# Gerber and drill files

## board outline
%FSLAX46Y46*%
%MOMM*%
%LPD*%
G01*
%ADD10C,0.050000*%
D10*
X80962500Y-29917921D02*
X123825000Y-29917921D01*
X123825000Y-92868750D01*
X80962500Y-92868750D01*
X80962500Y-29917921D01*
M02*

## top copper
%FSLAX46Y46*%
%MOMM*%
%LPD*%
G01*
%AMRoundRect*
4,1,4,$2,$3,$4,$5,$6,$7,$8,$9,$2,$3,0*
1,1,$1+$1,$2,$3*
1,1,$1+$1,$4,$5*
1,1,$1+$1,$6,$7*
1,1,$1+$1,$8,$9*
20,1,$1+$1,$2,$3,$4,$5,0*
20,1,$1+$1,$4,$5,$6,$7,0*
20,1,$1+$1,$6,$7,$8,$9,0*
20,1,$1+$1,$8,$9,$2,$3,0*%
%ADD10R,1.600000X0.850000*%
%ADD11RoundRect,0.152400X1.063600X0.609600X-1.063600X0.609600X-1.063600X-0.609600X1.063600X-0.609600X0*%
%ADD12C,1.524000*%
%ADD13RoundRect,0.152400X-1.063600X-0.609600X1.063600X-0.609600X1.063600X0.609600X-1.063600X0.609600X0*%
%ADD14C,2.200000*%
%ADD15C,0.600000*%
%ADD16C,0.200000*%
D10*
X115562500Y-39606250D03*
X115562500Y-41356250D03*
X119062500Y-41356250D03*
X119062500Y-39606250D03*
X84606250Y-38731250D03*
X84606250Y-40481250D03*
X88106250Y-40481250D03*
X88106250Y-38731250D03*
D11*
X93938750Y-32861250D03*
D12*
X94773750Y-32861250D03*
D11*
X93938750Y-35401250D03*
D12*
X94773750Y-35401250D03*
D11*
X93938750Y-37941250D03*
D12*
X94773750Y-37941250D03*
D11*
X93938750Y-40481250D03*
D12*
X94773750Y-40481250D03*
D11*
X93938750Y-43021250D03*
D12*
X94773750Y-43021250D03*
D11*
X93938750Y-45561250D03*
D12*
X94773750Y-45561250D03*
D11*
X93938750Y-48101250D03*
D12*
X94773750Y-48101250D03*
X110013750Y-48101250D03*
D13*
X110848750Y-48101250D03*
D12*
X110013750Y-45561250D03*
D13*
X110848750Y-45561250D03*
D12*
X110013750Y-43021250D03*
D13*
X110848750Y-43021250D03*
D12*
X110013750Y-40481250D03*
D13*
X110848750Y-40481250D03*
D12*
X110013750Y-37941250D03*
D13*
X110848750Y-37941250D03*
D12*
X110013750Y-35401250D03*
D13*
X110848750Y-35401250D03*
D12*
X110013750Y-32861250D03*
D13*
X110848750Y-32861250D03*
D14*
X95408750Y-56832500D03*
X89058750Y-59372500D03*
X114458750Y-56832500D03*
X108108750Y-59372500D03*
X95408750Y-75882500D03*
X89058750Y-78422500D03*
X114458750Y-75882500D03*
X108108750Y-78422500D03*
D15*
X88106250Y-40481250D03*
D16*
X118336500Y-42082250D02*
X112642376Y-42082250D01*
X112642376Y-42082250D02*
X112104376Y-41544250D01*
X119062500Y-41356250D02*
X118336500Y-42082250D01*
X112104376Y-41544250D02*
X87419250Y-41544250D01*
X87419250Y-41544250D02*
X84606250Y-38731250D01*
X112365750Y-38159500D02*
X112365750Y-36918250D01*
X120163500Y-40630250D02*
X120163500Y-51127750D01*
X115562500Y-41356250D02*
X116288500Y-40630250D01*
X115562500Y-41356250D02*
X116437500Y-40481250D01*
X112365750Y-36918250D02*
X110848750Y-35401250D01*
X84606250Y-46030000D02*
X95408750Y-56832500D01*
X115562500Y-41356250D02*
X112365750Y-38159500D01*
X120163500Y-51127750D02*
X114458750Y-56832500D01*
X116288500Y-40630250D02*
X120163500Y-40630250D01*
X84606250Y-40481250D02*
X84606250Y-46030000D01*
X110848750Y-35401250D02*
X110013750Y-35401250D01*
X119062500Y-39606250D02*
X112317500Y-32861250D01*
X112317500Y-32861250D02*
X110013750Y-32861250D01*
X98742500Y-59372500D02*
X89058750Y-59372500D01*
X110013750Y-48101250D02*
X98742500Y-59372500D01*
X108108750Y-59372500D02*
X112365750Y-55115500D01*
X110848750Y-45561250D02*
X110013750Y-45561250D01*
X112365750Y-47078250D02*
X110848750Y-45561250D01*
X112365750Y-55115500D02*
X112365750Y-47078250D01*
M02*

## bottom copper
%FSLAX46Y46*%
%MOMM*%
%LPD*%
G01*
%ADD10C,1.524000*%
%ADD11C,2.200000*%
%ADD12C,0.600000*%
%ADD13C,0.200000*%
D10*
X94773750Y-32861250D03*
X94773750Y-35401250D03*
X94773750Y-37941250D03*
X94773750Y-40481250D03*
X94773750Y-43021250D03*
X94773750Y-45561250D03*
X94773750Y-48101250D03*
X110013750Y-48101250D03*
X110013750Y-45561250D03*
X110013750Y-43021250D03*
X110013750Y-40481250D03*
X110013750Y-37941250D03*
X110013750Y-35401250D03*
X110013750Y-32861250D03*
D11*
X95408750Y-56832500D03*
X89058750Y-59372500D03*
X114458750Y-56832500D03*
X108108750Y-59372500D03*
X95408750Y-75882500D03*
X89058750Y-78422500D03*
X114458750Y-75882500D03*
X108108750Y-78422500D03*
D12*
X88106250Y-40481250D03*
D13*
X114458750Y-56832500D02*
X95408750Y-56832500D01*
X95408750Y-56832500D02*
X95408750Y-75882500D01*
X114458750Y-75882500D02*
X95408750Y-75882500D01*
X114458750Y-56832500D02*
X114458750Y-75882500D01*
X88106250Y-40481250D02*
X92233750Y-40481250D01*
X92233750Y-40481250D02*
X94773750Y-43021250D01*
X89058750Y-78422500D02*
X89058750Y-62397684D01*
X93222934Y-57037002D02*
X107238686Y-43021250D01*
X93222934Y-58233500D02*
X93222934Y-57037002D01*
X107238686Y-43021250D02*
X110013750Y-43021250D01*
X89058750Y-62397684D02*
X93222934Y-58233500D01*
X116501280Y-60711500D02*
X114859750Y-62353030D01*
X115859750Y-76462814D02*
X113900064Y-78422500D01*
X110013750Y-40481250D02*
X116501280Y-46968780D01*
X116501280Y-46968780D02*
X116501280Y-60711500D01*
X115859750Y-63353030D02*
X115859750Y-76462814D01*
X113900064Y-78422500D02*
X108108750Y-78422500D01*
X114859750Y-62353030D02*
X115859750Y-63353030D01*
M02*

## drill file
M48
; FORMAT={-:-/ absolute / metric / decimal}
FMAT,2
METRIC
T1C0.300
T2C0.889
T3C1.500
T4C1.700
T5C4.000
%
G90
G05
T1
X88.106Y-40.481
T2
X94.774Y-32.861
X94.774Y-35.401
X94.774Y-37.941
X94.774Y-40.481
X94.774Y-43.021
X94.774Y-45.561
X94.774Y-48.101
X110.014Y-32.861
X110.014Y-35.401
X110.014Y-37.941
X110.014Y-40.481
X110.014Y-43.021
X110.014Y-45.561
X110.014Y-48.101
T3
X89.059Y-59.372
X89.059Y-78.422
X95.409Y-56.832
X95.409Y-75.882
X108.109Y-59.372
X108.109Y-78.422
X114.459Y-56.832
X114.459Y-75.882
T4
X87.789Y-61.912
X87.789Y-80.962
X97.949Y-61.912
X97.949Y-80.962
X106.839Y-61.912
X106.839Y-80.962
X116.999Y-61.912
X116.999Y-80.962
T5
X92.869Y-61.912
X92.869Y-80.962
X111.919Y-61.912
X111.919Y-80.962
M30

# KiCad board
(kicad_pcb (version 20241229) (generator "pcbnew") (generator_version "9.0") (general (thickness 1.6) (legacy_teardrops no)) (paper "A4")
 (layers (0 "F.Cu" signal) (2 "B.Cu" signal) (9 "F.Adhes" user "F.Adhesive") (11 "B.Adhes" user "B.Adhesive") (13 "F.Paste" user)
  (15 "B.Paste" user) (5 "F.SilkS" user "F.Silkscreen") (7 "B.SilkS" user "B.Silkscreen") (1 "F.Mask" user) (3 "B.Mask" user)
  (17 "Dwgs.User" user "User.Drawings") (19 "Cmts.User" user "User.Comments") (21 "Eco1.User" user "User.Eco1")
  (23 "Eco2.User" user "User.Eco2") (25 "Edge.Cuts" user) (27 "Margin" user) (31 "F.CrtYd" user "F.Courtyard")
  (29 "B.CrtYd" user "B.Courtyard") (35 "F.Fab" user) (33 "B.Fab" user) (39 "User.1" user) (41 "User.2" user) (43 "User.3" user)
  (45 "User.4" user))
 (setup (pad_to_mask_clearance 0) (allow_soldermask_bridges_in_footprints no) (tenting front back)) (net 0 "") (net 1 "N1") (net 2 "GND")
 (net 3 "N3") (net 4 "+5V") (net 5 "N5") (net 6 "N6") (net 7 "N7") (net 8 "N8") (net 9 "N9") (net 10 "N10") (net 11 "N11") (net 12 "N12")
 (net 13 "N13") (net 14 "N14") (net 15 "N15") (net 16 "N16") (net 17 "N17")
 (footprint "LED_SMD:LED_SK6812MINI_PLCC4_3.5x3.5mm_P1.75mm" (layer "F.Cu") (at 117.3125 40.48125)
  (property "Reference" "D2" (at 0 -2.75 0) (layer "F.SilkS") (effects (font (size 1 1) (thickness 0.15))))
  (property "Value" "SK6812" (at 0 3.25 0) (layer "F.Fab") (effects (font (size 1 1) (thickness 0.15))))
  (pad "1" smd rect (at -1.75 -0.875) (size 1.6 0.85) (layers "F.Cu" "F.Mask" "F.Paste") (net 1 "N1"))
  (pad "2" smd rect (at -1.75 0.875) (size 1.6 0.85) (layers "F.Cu" "F.Mask" "F.Paste") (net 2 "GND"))
  (pad "3" smd rect (at 1.75 0.875) (size 1.6 0.85) (layers "F.Cu" "F.Mask" "F.Paste") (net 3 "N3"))
  (pad "4" smd rect (at 1.75 -0.875) (size 1.6 0.85) (layers "F.Cu" "F.Mask" "F.Paste") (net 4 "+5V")))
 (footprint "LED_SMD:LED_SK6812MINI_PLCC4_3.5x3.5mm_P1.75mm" (layer "F.Cu") (at 86.35625 39.60625)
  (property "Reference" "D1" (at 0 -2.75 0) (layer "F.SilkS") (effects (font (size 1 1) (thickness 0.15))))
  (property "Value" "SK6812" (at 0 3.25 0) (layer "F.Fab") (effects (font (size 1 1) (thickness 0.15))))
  (pad "1" smd rect (at -1.75 -0.875) (size 1.6 0.85) (layers "F.Cu" "F.Mask" "F.Paste") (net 3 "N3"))
  (pad "2" smd rect (at -1.75 0.875) (size 1.6 0.85) (layers "F.Cu" "F.Mask" "F.Paste") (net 2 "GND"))
  (pad "3" smd rect (at 1.75 0.875) (size 1.6 0.85) (layers "F.Cu" "F.Mask" "F.Paste") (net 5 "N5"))
  (pad "4" smd rect (at 1.75 -0.875) (size 1.6 0.85) (layers "F.Cu" "F.Mask" "F.Paste") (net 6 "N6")))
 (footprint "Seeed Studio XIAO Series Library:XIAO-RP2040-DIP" (layer "F.Cu") (at 102.39375 40.48125)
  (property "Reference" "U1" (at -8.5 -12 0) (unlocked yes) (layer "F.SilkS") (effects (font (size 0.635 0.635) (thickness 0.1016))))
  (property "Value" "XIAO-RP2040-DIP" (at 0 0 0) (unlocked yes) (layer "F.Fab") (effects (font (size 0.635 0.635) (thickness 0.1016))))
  (pad "1" smd roundrect (at -8.455 -7.62 180) (size 2.432 1.524) (layers "F.Cu" "F.Mask") (roundrect_rratio 0.1) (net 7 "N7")
   (thermal_bridge_angle 45))
  (pad "1" thru_hole circle (at -7.62 -7.62 180) (size 1.524 1.524) (drill 0.889) (layers "*.Cu" "*.Mask") (remove_unused_layers no)
   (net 7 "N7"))
  (pad "2" smd roundrect (at -8.455 -5.08 180) (size 2.432 1.524) (layers "F.Cu" "F.Mask") (roundrect_rratio 0.1) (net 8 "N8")
   (thermal_bridge_angle 45))
  (pad "2" thru_hole circle (at -7.62 -5.08 180) (size 1.524 1.524) (drill 0.889) (layers "*.Cu" "*.Mask") (remove_unused_layers no)
   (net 8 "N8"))
  (pad "3" smd roundrect (at -8.455 -2.54 180) (size 2.432 1.524) (layers "F.Cu" "F.Mask") (roundrect_rratio 0.1) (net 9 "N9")
   (thermal_bridge_angle 45))
  (pad "3" thru_hole circle (at -7.62 -2.54 180) (size 1.524 1.524) (drill 0.889) (layers "*.Cu" "*.Mask") (remove_unused_layers no)
   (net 9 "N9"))
  (pad "4" smd roundrect (at -8.455 0 180) (size 2.432 1.524) (layers "F.Cu" "F.Mask") (roundrect_rratio 0.1) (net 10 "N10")
   (thermal_bridge_angle 45))
  (pad "4" thru_hole circle (at -7.62 0 180) (size 1.524 1.524) (drill 0.889) (layers "*.Cu" "*.Mask") (remove_unused_layers no)
   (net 10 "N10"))
  (pad "5" smd roundrect (at -8.455 2.54 180) (size 2.432 1.524) (layers "F.Cu" "F.Mask") (roundrect_rratio 0.1) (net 5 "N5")
   (thermal_bridge_angle 45))
  (pad "5" thru_hole circle (at -7.62 2.54 180) (size 1.524 1.524) (drill 0.889) (layers "*.Cu" "*.Mask") (remove_unused_layers no)
   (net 5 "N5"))
  (pad "6" smd roundrect (at -8.455 5.08 180) (size 2.432 1.524) (layers "F.Cu" "F.Mask") (roundrect_rratio 0.1) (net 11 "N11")
   (thermal_bridge_angle 45))
  (pad "6" thru_hole circle (at -7.62 5.08 180) (size 1.524 1.524) (drill 0.889) (layers "*.Cu" "*.Mask") (remove_unused_layers no)
   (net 11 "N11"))
  (pad "7" smd roundrect (at -8.455 7.62 180) (size 2.432 1.524) (layers "F.Cu" "F.Mask") (roundrect_rratio 0.1) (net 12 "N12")
   (thermal_bridge_angle 45))
  (pad "7" thru_hole circle (at -7.62 7.62 180) (size 1.524 1.524) (drill 0.889) (layers "*.Cu" "*.Mask") (remove_unused_layers no)
   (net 12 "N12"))
  (pad "8" thru_hole circle (at 7.62 7.62) (size 1.524 1.524) (drill 0.889) (layers "*.Cu" "*.Mask") (remove_unused_layers no)
   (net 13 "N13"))
  (pad "8" smd roundrect (at 8.455 7.62) (size 2.432 1.524) (layers "F.Cu" "F.Mask") (roundrect_rratio 0.1) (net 13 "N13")
   (thermal_bridge_angle 45))
  (pad "9" thru_hole circle (at 7.62 5.08) (size 1.524 1.524) (drill 0.889) (layers "*.Cu" "*.Mask") (remove_unused_layers no)
   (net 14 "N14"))
  (pad "9" smd roundrect (at 8.455 5.08) (size 2.432 1.524) (layers "F.Cu" "F.Mask") (roundrect_rratio 0.1) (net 14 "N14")
   (thermal_bridge_angle 45))
  (pad "10" thru_hole circle (at 7.62 2.54) (size 1.524 1.524) (drill 0.889) (layers "*.Cu" "*.Mask") (remove_unused_layers no)
   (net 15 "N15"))
  (pad "10" smd roundrect (at 8.455 2.54) (size 2.432 1.524) (layers "F.Cu" "F.Mask") (roundrect_rratio 0.1) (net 15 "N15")
   (thermal_bridge_angle 45))
  (pad "11" thru_hole circle (at 7.62 0) (size 1.524 1.524) (drill 0.889) (layers "*.Cu" "*.Mask") (remove_unused_layers no) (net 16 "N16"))
  (pad "11" smd roundrect (at 8.455 0) (size 2.432 1.524) (layers "F.Cu" "F.Mask") (roundrect_rratio 0.1) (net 16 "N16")
   (thermal_bridge_angle 45))
  (pad "12" thru_hole circle (at 7.62 -2.54) (size 1.524 1.524) (drill 0.889) (layers "*.Cu" "*.Mask") (remove_unused_layers no)
   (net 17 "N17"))
  (pad "12" smd roundrect (at 8.455 -2.54) (size 2.432 1.524) (layers "F.Cu" "F.Mask") (roundrect_rratio 0.1) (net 17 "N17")
   (thermal_bridge_angle 45))
  (pad "13" thru_hole circle (at 7.62 -5.08) (size 1.524 1.524) (drill 0.889) (layers "*.Cu" "*.Mask") (remove_unused_layers no)
   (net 2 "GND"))
  (pad "13" smd roundrect (at 8.455 -5.08) (size 2.432 1.524) (layers "F.Cu" "F.Mask") (roundrect_rratio 0.1) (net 2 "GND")
   (thermal_bridge_angle 45))
  (pad "14" thru_hole circle (at 7.62 -7.62) (size 1.524 1.524) (drill 0.889) (layers "*.Cu" "*.Mask") (remove_unused_layers no)
   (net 4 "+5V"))
  (pad "14" smd roundrect (at 8.455 -7.62) (size 2.432 1.524) (layers "F.Cu" "F.Mask") (roundrect_rratio 0.1) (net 4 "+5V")
   (thermal_bridge_angle 45)))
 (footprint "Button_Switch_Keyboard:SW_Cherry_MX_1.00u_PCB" (layer "F.Cu") (at 95.40875 56.8325)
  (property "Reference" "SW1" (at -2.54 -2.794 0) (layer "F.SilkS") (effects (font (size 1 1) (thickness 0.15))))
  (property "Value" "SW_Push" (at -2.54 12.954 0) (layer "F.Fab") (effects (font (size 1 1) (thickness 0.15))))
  (pad "" np_thru_hole circle (at -7.62 5.08) (size 1.7 1.7) (drill 1.7) (layers "*.Cu" "*.Mask"))
  (pad "" np_thru_hole circle (at -2.54 5.08) (size 4 4) (drill 4) (layers "*.Cu" "*.Mask"))
  (pad "" np_thru_hole circle (at 2.54 5.08) (size 1.7 1.7) (drill 1.7) (layers "*.Cu" "*.Mask"))
  (pad "1" thru_hole circle (at 0 0) (size 2.2 2.2) (drill 1.5) (layers "*.Cu" "*.Mask") (remove_unused_layers no) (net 2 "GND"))
  (pad "2" thru_hole circle (at -6.35 2.54) (size 2.2 2.2) (drill 1.5) (layers "*.Cu" "*.Mask") (remove_unused_layers no) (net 13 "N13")))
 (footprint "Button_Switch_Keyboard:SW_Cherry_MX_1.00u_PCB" (layer "F.Cu") (at 114.45875 56.8325)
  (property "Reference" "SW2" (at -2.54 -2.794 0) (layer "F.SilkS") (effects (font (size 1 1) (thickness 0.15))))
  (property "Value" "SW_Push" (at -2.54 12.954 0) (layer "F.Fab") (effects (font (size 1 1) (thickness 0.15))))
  (pad "" np_thru_hole circle (at -7.62 5.08) (size 1.7 1.7) (drill 1.7) (layers "*.Cu" "*.Mask"))
  (pad "" np_thru_hole circle (at -2.54 5.08) (size 4 4) (drill 4) (layers "*.Cu" "*.Mask"))
  (pad "" np_thru_hole circle (at 2.54 5.08) (size 1.7 1.7) (drill 1.7) (layers "*.Cu" "*.Mask"))
  (pad "1" thru_hole circle (at 0 0) (size 2.2 2.2) (drill 1.5) (layers "*.Cu" "*.Mask") (remove_unused_layers no) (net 2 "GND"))
  (pad "2" thru_hole circle (at -6.35 2.54) (size 2.2 2.2) (drill 1.5) (layers "*.Cu" "*.Mask") (remove_unused_layers no) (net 14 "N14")))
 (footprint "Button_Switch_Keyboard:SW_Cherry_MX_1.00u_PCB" (layer "F.Cu") (at 95.40875 75.8825)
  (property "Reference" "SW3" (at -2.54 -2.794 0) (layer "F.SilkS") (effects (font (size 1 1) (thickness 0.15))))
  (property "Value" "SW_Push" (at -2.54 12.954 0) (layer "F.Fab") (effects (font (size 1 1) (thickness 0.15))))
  (pad "" np_thru_hole circle (at -7.62 5.08) (size 1.7 1.7) (drill 1.7) (layers "*.Cu" "*.Mask"))
  (pad "" np_thru_hole circle (at -2.54 5.08) (size 4 4) (drill 4) (layers "*.Cu" "*.Mask"))
  (pad "" np_thru_hole circle (at 2.54 5.08) (size 1.7 1.7) (drill 1.7) (layers "*.Cu" "*.Mask"))
  (pad "1" thru_hole circle (at 0 0) (size 2.2 2.2) (drill 1.5) (layers "*.Cu" "*.Mask") (remove_unused_layers no) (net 2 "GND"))
  (pad "2" thru_hole circle (at -6.35 2.54) (size 2.2 2.2) (drill 1.5) (layers "*.Cu" "*.Mask") (remove_unused_layers no) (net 15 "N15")))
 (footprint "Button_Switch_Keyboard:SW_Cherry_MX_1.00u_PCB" (layer "F.Cu") (at 114.45875 75.8825)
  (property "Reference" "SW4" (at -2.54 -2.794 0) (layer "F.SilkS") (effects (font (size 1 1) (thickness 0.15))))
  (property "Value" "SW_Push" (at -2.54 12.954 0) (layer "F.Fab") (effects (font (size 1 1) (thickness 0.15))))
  (pad "" np_thru_hole circle (at -7.62 5.08) (size 1.7 1.7) (drill 1.7) (layers "*.Cu" "*.Mask"))
  (pad "" np_thru_hole circle (at -2.54 5.08) (size 4 4) (drill 4) (layers "*.Cu" "*.Mask"))
  (pad "" np_thru_hole circle (at 2.54 5.08) (size 1.7 1.7) (drill 1.7) (layers "*.Cu" "*.Mask"))
  (pad "1" thru_hole circle (at 0 0) (size 2.2 2.2) (drill 1.5) (layers "*.Cu" "*.Mask") (remove_unused_layers no) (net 2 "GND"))
  (pad "2" thru_hole circle (at -6.35 2.54) (size 2.2 2.2) (drill 1.5) (layers "*.Cu" "*.Mask") (remove_unused_layers no) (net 16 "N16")))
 (gr_rect (start 80.9625 29.917921) (end 123.825 92.86875) (stroke (width 0.05) (type default)) (fill no) (layer "Edge.Cuts"))
 (segment (start 118.3365 42.08225) (end 112.642376 42.08225) (width 0.2) (layer "F.Cu") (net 3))
 (segment (start 112.642376 42.08225) (end 112.104376 41.54425) (width 0.2) (layer "F.Cu") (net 3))
 (segment (start 119.0625 41.35625) (end 118.3365 42.08225) (width 0.2) (layer "F.Cu") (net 3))
 (segment (start 112.104376 41.54425) (end 87.41925 41.54425) (width 0.2) (layer "F.Cu") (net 3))
 (segment (start 87.41925 41.54425) (end 84.60625 38.73125) (width 0.2) (layer "F.Cu") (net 3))
 (segment (start 112.36575 38.1595) (end 112.36575 36.91825) (width 0.2) (layer "F.Cu") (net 2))
 (segment (start 120.1635 40.63025) (end 120.1635 51.12775) (width 0.2) (layer "F.Cu") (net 2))
 (segment (start 115.5625 41.35625) (end 116.2885 40.63025) (width 0.2) (layer "F.Cu") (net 2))
 (segment (start 115.5625 41.35625) (end 116.4375 40.48125) (width 0.2) (layer "F.Cu") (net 2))
 (segment (start 112.36575 36.91825) (end 110.84875 35.40125) (width 0.2) (layer "F.Cu") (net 2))
 (segment (start 84.60625 46.03) (end 95.40875 56.8325) (width 0.2) (layer "F.Cu") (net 2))
 (segment (start 115.5625 41.35625) (end 112.36575 38.1595) (width 0.2) (layer "F.Cu") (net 2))
 (segment (start 120.1635 51.12775) (end 114.45875 56.8325) (width 0.2) (layer "F.Cu") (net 2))
 (segment (start 116.2885 40.63025) (end 120.1635 40.63025) (width 0.2) (layer "F.Cu") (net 2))
 (segment (start 84.60625 40.48125) (end 84.60625 46.03) (width 0.2) (layer "F.Cu") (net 2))
 (segment (start 110.84875 35.40125) (end 110.01375 35.40125) (width 0.2) (layer "F.Cu") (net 2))
 (segment (start 114.45875 56.8325) (end 95.40875 56.8325) (width 0.2) (layer "B.Cu") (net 2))
 (segment (start 95.40875 56.8325) (end 95.40875 75.8825) (width 0.2) (layer "B.Cu") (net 2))
 (segment (start 114.45875 75.8825) (end 95.40875 75.8825) (width 0.2) (layer "B.Cu") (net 2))
 (segment (start 114.45875 56.8325) (end 114.45875 75.8825) (width 0.2) (layer "B.Cu") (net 2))
 (via (at 88.10625 40.48125) (size 0.6) (drill 0.3) (layers "F.Cu" "B.Cu") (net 5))
 (segment (start 88.10625 40.48125) (end 92.23375 40.48125) (width 0.2) (layer "B.Cu") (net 5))
 (segment (start 92.23375 40.48125) (end 94.77375 43.02125) (width 0.2) (layer "B.Cu") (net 5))
 (segment (start 119.0625 39.60625) (end 112.3175 32.86125) (width 0.2) (layer "F.Cu") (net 4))
 (segment (start 112.3175 32.86125) (end 110.01375 32.86125) (width 0.2) (layer "F.Cu") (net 4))
 (segment (start 98.7425 59.3725) (end 89.05875 59.3725) (width 0.2) (layer "F.Cu") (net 13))
 (segment (start 110.01375 48.10125) (end 98.7425 59.3725) (width 0.2) (layer "F.Cu") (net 13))
 (segment (start 108.10875 59.3725) (end 112.36575 55.1155) (width 0.2) (layer "F.Cu") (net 14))
 (segment (start 110.84875 45.56125) (end 110.01375 45.56125) (width 0.2) (layer "F.Cu") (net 14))
 (segment (start 112.36575 47.07825) (end 110.84875 45.56125) (width 0.2) (layer "F.Cu") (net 14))
 (segment (start 112.36575 55.1155) (end 112.36575 47.07825) (width 0.2) (layer "F.Cu") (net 14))
 (segment (start 89.05875 78.4225) (end 89.05875 62.397684) (width 0.2) (layer "B.Cu") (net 15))
 (segment (start 93.222934 57.037002) (end 107.238686 43.02125) (width 0.2) (layer "B.Cu") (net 15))
 (segment (start 93.222934 58.2335) (end 93.222934 57.037002) (width 0.2) (layer "B.Cu") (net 15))
 (segment (start 107.238686 43.02125) (end 110.01375 43.02125) (width 0.2) (layer "B.Cu") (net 15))
 (segment (start 89.05875 62.397684) (end 93.222934 58.2335) (width 0.2) (layer "B.Cu") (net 15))
 (segment (start 116.50128 60.7115) (end 114.85975 62.35303) (width 0.2) (layer "B.Cu") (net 16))
 (segment (start 115.85975 76.462814) (end 113.900064 78.4225) (width 0.2) (layer "B.Cu") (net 16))
 (segment (start 110.01375 40.48125) (end 116.50128 46.96878) (width 0.2) (layer "B.Cu") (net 16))
 (segment (start 116.50128 46.96878) (end 116.50128 60.7115) (width 0.2) (layer "B.Cu") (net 16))
 (segment (start 115.85975 63.35303) (end 115.85975 76.462814) (width 0.2) (layer "B.Cu") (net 16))
 (segment (start 113.900064 78.4225) (end 108.10875 78.4225) (width 0.2) (layer "B.Cu") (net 16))
 (segment (start 114.85975 62.35303) (end 115.85975 63.35303) (width 0.2) (layer "B.Cu") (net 16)))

